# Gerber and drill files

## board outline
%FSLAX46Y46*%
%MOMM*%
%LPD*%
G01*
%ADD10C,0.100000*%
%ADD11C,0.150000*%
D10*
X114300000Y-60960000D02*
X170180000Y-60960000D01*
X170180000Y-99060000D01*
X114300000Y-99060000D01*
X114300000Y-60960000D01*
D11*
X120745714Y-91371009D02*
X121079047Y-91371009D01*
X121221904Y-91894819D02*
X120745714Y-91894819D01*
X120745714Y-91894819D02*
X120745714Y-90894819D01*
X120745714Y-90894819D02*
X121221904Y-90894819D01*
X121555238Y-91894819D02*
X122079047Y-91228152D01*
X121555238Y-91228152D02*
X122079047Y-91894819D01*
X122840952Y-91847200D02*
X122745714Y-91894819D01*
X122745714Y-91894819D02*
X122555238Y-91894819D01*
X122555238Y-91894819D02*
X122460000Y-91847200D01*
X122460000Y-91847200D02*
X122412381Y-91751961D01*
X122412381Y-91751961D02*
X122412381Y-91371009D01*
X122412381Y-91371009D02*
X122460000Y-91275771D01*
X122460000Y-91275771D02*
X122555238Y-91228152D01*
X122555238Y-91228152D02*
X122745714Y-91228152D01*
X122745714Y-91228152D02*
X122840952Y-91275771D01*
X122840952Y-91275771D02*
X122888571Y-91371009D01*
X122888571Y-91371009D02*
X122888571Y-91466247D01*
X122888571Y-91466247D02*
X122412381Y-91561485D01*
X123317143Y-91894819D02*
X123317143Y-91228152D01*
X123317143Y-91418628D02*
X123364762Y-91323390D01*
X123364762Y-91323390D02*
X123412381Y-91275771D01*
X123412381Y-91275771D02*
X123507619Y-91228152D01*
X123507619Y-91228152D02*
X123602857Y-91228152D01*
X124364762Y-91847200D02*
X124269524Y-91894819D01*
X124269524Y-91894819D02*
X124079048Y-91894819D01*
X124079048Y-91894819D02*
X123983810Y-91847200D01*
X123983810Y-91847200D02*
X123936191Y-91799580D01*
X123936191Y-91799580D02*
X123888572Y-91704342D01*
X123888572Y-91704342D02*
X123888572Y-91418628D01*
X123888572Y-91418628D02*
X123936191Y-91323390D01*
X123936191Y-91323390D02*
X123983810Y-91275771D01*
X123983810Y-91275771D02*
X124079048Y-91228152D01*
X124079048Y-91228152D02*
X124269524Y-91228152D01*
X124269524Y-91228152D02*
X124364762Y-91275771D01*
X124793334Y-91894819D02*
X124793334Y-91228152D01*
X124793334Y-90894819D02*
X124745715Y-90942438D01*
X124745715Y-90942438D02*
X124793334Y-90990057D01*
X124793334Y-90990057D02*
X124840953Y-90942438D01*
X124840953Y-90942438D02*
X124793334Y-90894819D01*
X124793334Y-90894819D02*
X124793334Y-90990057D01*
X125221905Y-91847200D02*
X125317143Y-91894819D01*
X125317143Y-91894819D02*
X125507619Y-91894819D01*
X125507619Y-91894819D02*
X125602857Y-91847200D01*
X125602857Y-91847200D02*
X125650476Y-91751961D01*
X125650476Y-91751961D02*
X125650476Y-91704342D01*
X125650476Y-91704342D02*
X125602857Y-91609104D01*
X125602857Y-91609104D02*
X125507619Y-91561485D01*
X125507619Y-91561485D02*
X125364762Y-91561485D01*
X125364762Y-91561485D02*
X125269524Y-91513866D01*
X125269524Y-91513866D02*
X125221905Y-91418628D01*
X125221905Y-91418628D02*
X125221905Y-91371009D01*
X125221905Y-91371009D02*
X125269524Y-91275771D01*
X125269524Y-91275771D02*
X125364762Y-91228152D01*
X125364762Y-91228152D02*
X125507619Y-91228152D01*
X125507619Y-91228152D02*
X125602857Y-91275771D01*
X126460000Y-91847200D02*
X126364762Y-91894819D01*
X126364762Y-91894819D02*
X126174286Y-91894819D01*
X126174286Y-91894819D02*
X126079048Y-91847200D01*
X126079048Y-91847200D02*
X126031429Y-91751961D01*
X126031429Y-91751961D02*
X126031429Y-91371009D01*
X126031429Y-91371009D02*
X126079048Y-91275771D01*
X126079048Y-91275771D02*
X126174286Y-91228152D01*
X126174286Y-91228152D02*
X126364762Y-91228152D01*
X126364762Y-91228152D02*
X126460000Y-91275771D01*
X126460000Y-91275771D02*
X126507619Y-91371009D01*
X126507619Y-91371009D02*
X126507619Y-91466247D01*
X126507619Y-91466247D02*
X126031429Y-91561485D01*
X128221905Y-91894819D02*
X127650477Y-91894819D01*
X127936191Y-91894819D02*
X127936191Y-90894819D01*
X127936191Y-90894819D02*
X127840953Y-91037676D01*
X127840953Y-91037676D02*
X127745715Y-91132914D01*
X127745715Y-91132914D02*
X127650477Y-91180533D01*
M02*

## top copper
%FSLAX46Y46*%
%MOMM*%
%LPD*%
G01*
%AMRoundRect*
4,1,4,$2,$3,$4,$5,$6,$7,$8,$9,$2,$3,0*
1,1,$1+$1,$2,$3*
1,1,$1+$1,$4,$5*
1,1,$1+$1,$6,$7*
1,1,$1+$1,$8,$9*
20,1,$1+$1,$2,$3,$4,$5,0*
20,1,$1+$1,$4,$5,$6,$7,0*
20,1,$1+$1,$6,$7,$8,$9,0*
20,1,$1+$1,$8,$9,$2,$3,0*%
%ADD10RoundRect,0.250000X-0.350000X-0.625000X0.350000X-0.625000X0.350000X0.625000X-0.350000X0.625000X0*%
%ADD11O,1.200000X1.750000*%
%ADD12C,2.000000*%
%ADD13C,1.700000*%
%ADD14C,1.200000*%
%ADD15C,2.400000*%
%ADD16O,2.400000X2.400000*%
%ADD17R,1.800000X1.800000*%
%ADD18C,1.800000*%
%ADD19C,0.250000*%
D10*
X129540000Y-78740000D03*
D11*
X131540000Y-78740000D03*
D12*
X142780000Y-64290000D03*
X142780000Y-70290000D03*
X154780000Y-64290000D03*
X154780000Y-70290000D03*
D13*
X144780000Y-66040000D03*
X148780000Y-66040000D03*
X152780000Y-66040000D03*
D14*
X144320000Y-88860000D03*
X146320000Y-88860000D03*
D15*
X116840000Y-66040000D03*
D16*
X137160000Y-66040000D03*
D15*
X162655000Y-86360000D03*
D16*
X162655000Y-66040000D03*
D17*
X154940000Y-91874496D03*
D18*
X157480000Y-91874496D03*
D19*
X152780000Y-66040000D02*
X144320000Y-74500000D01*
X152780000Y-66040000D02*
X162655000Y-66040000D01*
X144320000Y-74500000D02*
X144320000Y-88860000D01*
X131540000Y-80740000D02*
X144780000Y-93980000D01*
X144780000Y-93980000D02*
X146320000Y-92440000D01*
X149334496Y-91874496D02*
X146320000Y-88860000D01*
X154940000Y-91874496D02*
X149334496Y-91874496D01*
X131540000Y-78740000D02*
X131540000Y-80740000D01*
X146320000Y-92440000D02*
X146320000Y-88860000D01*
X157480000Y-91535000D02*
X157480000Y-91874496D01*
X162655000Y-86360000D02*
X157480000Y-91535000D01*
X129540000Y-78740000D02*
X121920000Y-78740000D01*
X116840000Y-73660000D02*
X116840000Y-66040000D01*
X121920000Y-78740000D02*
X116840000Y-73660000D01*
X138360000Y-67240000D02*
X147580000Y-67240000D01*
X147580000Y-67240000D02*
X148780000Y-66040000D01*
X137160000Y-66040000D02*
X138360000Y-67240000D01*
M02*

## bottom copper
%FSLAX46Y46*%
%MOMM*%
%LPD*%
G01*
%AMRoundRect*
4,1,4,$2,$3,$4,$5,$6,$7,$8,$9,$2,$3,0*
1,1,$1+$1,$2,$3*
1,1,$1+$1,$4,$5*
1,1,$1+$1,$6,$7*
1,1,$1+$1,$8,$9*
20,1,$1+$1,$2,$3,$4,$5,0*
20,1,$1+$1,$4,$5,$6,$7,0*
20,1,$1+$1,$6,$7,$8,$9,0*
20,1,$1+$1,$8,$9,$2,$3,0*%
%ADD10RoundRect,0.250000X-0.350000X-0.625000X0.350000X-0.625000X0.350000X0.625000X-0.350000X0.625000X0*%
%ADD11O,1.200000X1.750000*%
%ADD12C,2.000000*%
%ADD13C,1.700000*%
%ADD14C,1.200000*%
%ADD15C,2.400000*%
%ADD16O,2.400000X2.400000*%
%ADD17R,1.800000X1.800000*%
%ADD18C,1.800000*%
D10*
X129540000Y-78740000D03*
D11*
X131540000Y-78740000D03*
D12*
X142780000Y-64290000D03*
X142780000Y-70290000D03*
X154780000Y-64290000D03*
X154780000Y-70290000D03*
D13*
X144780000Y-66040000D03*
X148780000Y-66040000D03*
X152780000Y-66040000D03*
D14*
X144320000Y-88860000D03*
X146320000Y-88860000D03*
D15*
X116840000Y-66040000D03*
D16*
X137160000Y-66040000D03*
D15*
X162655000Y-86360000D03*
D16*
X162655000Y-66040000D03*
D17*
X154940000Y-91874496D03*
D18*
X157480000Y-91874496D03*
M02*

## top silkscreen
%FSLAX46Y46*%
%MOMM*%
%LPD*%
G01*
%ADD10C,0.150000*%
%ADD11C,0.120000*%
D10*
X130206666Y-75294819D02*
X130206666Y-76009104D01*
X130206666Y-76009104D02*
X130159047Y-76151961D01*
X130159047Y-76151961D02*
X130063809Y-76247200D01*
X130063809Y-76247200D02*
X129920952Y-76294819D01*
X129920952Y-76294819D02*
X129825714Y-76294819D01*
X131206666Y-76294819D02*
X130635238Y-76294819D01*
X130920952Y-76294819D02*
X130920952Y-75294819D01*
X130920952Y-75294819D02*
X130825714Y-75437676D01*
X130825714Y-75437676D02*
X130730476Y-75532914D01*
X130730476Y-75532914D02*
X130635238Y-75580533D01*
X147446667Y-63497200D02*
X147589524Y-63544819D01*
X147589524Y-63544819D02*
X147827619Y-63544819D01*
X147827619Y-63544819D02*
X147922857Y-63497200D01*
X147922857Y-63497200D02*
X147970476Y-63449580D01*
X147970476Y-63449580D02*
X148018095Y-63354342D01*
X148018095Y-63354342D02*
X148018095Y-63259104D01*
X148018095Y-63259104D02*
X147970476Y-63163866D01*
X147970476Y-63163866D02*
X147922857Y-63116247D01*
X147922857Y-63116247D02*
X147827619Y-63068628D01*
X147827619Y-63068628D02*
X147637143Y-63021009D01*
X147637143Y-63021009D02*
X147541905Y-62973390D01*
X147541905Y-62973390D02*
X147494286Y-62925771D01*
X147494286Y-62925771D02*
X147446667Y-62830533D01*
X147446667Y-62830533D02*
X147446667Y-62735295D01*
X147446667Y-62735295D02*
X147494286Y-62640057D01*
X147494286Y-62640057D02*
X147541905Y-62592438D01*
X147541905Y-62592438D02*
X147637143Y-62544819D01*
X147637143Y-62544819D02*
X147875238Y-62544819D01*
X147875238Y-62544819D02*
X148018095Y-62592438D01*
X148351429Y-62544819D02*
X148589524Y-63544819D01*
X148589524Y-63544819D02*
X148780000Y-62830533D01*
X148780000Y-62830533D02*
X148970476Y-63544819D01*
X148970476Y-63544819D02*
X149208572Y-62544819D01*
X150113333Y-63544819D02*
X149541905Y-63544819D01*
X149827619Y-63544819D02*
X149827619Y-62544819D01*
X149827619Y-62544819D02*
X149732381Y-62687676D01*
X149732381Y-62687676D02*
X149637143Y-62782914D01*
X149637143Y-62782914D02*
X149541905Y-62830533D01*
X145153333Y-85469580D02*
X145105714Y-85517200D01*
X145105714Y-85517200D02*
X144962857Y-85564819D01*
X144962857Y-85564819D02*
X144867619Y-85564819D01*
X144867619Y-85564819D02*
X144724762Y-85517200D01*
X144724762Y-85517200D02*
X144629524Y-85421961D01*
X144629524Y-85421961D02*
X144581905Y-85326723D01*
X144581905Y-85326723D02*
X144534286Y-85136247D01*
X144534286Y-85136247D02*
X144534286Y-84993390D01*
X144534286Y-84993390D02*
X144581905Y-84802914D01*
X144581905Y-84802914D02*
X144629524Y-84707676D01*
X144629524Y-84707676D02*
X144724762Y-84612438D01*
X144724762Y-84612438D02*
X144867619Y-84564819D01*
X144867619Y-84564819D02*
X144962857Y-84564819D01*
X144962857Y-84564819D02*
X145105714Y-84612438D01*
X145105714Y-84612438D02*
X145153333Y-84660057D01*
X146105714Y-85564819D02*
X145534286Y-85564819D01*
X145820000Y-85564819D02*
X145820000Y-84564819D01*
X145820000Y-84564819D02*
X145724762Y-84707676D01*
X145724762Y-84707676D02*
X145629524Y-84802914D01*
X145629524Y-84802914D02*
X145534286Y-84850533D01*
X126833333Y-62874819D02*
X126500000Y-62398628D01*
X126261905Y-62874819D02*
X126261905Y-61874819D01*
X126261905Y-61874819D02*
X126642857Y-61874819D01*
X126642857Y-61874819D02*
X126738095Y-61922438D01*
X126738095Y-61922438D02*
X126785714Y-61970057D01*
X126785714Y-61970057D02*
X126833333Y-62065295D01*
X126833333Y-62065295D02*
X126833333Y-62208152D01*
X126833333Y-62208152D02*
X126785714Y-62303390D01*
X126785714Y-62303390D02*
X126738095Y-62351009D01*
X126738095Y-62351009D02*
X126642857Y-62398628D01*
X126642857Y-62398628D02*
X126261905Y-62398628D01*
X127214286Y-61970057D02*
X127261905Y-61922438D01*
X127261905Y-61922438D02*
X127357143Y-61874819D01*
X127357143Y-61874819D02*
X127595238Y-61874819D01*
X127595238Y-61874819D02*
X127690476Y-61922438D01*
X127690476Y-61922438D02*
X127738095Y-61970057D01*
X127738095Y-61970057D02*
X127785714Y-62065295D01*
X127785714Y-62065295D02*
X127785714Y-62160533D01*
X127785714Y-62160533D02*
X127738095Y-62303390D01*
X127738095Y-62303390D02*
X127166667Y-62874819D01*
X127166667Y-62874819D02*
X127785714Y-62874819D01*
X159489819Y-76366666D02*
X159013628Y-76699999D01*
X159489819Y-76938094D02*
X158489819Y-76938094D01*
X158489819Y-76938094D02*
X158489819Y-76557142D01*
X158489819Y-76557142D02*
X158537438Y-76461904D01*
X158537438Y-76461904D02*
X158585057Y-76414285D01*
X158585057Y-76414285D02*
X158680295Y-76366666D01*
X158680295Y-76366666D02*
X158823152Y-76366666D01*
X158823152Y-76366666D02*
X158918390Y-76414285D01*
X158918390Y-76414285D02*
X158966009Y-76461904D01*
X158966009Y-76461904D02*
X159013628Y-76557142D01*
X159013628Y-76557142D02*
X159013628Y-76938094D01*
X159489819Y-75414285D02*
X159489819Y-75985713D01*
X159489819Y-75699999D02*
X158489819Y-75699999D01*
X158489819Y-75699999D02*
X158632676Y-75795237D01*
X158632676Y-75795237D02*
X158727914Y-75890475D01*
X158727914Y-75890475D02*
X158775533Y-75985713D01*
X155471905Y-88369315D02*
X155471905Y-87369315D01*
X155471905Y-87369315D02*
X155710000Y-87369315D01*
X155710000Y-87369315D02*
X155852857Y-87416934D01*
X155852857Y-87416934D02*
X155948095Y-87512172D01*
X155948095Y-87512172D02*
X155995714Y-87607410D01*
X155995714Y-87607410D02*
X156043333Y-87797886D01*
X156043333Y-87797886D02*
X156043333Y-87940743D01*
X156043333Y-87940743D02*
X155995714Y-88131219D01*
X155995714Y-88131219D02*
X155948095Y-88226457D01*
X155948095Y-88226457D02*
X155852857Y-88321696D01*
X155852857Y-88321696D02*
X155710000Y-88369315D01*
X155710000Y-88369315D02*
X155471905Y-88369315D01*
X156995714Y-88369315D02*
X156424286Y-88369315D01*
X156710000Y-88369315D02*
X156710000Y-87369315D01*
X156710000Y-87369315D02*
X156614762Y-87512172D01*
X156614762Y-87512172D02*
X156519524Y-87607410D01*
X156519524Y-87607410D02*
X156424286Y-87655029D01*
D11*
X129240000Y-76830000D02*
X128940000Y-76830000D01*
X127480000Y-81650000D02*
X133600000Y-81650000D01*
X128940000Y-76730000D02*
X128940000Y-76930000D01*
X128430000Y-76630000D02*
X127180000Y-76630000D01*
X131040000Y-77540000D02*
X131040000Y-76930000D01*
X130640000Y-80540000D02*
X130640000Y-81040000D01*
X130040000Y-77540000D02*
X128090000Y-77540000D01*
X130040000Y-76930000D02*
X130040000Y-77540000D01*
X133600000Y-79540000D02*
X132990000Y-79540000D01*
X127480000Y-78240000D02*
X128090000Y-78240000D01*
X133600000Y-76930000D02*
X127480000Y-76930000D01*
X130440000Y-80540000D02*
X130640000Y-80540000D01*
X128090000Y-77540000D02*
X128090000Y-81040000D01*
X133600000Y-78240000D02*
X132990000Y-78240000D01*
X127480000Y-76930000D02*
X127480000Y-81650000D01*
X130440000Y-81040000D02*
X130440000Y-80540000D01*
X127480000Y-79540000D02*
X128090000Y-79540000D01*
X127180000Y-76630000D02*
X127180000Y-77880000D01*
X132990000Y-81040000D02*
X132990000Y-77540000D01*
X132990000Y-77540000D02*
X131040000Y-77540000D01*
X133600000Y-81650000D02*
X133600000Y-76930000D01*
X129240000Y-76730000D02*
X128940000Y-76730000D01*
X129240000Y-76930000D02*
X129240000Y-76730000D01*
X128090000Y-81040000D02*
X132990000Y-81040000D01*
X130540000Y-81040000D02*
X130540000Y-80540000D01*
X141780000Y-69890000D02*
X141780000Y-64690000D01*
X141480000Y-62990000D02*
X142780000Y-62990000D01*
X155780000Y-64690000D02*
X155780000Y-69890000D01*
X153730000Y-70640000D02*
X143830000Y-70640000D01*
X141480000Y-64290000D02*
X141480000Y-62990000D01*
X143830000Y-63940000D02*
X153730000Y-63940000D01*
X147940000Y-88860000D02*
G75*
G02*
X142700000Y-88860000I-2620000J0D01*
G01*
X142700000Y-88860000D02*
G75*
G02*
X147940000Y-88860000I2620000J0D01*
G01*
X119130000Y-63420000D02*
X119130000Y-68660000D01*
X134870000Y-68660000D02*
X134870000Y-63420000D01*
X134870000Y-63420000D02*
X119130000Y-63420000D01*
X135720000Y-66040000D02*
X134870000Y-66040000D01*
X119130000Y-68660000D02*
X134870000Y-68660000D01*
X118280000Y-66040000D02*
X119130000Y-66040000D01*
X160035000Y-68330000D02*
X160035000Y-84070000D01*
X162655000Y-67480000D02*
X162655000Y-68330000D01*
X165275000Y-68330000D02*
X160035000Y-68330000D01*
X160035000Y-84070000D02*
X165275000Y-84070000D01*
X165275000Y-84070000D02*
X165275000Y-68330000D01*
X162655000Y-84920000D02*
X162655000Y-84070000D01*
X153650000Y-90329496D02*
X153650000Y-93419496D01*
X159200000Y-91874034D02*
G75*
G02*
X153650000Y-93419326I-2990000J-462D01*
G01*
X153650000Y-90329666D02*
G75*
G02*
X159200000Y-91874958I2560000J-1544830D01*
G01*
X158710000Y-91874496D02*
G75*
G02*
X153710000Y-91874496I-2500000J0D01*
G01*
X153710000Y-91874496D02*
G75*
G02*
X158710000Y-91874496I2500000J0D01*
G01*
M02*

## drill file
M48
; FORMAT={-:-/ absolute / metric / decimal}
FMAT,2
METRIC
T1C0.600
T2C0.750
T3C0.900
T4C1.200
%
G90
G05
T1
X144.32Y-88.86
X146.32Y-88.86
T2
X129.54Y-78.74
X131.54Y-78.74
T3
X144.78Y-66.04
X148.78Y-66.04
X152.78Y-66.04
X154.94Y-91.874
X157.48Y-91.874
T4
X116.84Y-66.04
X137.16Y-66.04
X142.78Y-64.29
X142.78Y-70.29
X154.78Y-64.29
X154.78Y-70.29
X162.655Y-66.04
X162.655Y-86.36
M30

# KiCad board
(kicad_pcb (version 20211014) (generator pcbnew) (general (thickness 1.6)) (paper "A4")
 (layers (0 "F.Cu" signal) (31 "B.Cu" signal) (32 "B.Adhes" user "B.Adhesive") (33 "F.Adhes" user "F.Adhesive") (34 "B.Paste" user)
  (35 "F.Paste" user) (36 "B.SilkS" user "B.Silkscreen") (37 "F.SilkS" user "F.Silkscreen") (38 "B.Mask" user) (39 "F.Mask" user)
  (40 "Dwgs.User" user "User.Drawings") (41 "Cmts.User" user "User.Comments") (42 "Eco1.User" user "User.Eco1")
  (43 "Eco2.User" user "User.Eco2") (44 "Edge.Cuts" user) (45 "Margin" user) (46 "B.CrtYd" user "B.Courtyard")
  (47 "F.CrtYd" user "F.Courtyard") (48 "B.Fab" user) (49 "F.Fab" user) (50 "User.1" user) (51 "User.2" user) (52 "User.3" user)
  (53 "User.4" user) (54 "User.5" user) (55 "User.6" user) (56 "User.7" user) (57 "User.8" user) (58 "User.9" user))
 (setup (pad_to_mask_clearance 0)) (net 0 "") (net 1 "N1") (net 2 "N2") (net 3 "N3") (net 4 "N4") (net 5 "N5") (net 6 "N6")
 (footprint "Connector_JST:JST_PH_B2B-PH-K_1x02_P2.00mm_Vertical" (layer "F.Cu") (at 129.54 78.74)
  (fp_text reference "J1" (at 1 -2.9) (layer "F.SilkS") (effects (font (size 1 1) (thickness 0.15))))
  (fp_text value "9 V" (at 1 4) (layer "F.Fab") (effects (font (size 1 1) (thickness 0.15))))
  (fp_line (start -0.3 -1.91) (end -0.6 -1.91) (layer "F.SilkS") (width 0.12))
  (fp_line (start -2.06 2.91) (end 4.06 2.91) (layer "F.SilkS") (width 0.12))
  (fp_line (start -0.6 -2.01) (end -0.6 -1.81) (layer "F.SilkS") (width 0.12))
  (fp_line (start -1.11 -2.11) (end -2.36 -2.11) (layer "F.SilkS") (width 0.12))
  (fp_line (start 1.5 -1.2) (end 1.5 -1.81) (layer "F.SilkS") (width 0.12))
  (fp_line (start 1.1 1.8) (end 1.1 2.3) (layer "F.SilkS") (width 0.12))
  (fp_line (start 0.5 -1.2) (end -1.45 -1.2) (layer "F.SilkS") (width 0.12))
  (fp_line (start 0.5 -1.81) (end 0.5 -1.2) (layer "F.SilkS") (width 0.12))
  (fp_line (start 4.06 0.8) (end 3.45 0.8) (layer "F.SilkS") (width 0.12))
  (fp_line (start -2.06 -0.5) (end -1.45 -0.5) (layer "F.SilkS") (width 0.12))
  (fp_line (start 4.06 -1.81) (end -2.06 -1.81) (layer "F.SilkS") (width 0.12))
  (fp_line (start 0.9 1.8) (end 1.1 1.8) (layer "F.SilkS") (width 0.12))
  (fp_line (start -1.45 -1.2) (end -1.45 2.3) (layer "F.SilkS") (width 0.12))
  (fp_line (start 4.06 -0.5) (end 3.45 -0.5) (layer "F.SilkS") (width 0.12))
  (fp_line (start -2.06 -1.81) (end -2.06 2.91) (layer "F.SilkS") (width 0.12))
  (fp_line (start 0.9 2.3) (end 0.9 1.8) (layer "F.SilkS") (width 0.12))
  (fp_line (start -2.06 0.8) (end -1.45 0.8) (layer "F.SilkS") (width 0.12))
  (fp_line (start -2.36 -2.11) (end -2.36 -0.86) (layer "F.SilkS") (width 0.12))
  (fp_line (start 3.45 2.3) (end 3.45 -1.2) (layer "F.SilkS") (width 0.12))
  (fp_line (start 3.45 -1.2) (end 1.5 -1.2) (layer "F.SilkS") (width 0.12))
  (fp_line (start 4.06 2.91) (end 4.06 -1.81) (layer "F.SilkS") (width 0.12))
  (fp_line (start -0.3 -2.01) (end -0.6 -2.01) (layer "F.SilkS") (width 0.12))
  (fp_line (start -0.3 -1.81) (end -0.3 -2.01) (layer "F.SilkS") (width 0.12))
  (fp_line (start -1.45 2.3) (end 3.45 2.3) (layer "F.SilkS") (width 0.12))
  (fp_line (start 1 2.3) (end 1 1.8) (layer "F.SilkS") (width 0.12))
  (pad "1" thru_hole roundrect (at 0 0) (size 1.2 1.75) (drill 0.75) (layers *.Cu *.Mask) (roundrect_rratio 0.208333) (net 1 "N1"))
  (pad "2" thru_hole oval (at 2 0) (size 1.2 1.75) (drill 0.75) (layers *.Cu *.Mask) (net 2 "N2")))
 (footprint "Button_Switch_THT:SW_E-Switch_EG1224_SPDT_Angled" (layer "F.Cu") (at 144.78 66.04)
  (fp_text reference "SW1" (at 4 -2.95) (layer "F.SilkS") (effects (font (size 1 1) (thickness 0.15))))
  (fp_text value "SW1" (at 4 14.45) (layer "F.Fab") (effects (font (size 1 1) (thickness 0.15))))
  (fp_line (start -3 3.85) (end -3 -1.35) (layer "F.SilkS") (width 0.12))
  (fp_line (start -3.3 -3.05) (end -2 -3.05) (layer "F.SilkS") (width 0.12))
  (fp_line (start 11 -1.35) (end 11 3.85) (layer "F.SilkS") (width 0.12))
  (fp_line (start 8.95 4.6) (end -0.95 4.6) (layer "F.SilkS") (width 0.12))
  (fp_line (start -3.3 -1.75) (end -3.3 -3.05) (layer "F.SilkS") (width 0.12))
  (fp_line (start -0.95 -2.1) (end 8.95 -2.1) (layer "F.SilkS") (width 0.12))
  (pad "" thru_hole circle (at -2 -1.75) (size 2 2) (drill 1.2) (layers *.Cu *.Mask))
  (pad "" thru_hole circle (at -2 4.25) (size 2 2) (drill 1.2) (layers *.Cu *.Mask))
  (pad "" thru_hole circle (at 10 -1.75) (size 2 2) (drill 1.2) (layers *.Cu *.Mask))
  (pad "" thru_hole circle (at 10 4.25) (size 2 2) (drill 1.2) (layers *.Cu *.Mask))
  (pad "1" thru_hole circle (at 0 0) (size 1.7 1.7) (drill 0.9) (layers *.Cu *.Mask) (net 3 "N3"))
  (pad "2" thru_hole circle (at 4 0) (size 1.7 1.7) (drill 0.9) (layers *.Cu *.Mask) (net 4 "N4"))
  (pad "3" thru_hole circle (at 8 0) (size 1.7 1.7) (drill 0.9) (layers *.Cu *.Mask) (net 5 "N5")))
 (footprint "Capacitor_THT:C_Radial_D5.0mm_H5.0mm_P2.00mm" (layer "F.Cu") (at 144.32 88.86)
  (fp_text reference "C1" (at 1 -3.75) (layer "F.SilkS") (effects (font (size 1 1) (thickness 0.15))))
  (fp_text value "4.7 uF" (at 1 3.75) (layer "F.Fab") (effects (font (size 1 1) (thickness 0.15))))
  (fp_circle (center 1 0) (end 3.62 0) (layer "F.SilkS") (width 0.12) (fill none))
  (pad "1" thru_hole circle (at 0 0) (size 1.2 1.2) (drill 0.6) (layers *.Cu *.Mask) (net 5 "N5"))
  (pad "2" thru_hole circle (at 2 0) (size 1.2 1.2) (drill 0.6) (layers *.Cu *.Mask) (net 2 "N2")))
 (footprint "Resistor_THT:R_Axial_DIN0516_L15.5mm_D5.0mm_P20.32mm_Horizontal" (layer "F.Cu") (at 116.84 66.04)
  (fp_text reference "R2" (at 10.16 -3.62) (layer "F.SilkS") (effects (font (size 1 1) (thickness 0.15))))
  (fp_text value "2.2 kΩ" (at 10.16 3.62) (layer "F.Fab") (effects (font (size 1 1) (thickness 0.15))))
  (fp_line (start 2.29 -2.62) (end 2.29 2.62) (layer "F.SilkS") (width 0.12))
  (fp_line (start 18.03 2.62) (end 18.03 -2.62) (layer "F.SilkS") (width 0.12))
  (fp_line (start 18.03 -2.62) (end 2.29 -2.62) (layer "F.SilkS") (width 0.12))
  (fp_line (start 18.88 0) (end 18.03 0) (layer "F.SilkS") (width 0.12))
  (fp_line (start 2.29 2.62) (end 18.03 2.62) (layer "F.SilkS") (width 0.12))
  (fp_line (start 1.44 0) (end 2.29 0) (layer "F.SilkS") (width 0.12))
  (pad "1" thru_hole circle (at 0 0) (size 2.4 2.4) (drill 1.2) (layers *.Cu *.Mask) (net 1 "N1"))
  (pad "2" thru_hole oval (at 20.32 0) (size 2.4 2.4) (drill 1.2) (layers *.Cu *.Mask) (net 4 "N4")))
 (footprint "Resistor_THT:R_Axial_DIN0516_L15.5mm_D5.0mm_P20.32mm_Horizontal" (layer "F.Cu") (at 162.655 86.36 90)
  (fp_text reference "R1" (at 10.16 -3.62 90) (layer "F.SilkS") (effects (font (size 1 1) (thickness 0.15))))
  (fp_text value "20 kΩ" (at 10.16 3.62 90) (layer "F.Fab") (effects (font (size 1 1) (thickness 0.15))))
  (fp_line (start 18.03 -2.62) (end 2.29 -2.62) (layer "F.SilkS") (width 0.12))
  (fp_line (start 18.88 0) (end 18.03 0) (layer "F.SilkS") (width 0.12))
  (fp_line (start 18.03 2.62) (end 18.03 -2.62) (layer "F.SilkS") (width 0.12))
  (fp_line (start 2.29 -2.62) (end 2.29 2.62) (layer "F.SilkS") (width 0.12))
  (fp_line (start 2.29 2.62) (end 18.03 2.62) (layer "F.SilkS") (width 0.12))
  (fp_line (start 1.44 0) (end 2.29 0) (layer "F.SilkS") (width 0.12))
  (pad "1" thru_hole circle (at 0 0 90) (size 2.4 2.4) (drill 1.2) (layers *.Cu *.Mask) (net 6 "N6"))
  (pad "2" thru_hole oval (at 20.32 0 90) (size 2.4 2.4) (drill 1.2) (layers *.Cu *.Mask) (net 5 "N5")))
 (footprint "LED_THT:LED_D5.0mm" (layer "F.Cu") (at 154.94 91.874496)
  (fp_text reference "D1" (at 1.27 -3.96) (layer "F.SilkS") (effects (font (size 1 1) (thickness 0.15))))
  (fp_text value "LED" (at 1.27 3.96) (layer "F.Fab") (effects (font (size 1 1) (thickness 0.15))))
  (fp_line (start -1.29 -1.545) (end -1.29 1.545) (layer "F.SilkS") (width 0.12))
  (fp_arc (start 4.26 -0.000462) (mid 2.072002 2.880433) (end -1.29 1.54483) (layer "F.SilkS") (width 0.12))
  (fp_arc (start -1.29 -1.54483) (mid 2.072002 -2.880433) (end 4.26 0.000462) (layer "F.SilkS") (width 0.12))
  (fp_circle (center 1.27 0) (end 3.77 0) (layer "F.SilkS") (width 0.12) (fill none))
  (pad "1" thru_hole rect (at 0 0) (size 1.8 1.8) (drill 0.9) (layers *.Cu *.Mask) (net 2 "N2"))
  (pad "2" thru_hole circle (at 2.54 0) (size 1.8 1.8) (drill 0.9) (layers *.Cu *.Mask) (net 6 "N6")))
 (gr_rect (start 170.18 99.06) (end 170.18 99.06) (layer "Edge.Cuts") (width 0.1) (fill none))
 (gr_rect (start 114.3 60.96) (end 170.18 99.06) (layer "Edge.Cuts") (width 0.1) (fill none))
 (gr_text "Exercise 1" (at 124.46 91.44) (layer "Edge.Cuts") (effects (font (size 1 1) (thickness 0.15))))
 (segment (start 152.78 66.04) (end 144.32 74.5) (width 0.25) (layer "F.Cu") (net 5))
 (segment (start 152.78 66.04) (end 162.655 66.04) (width 0.25) (layer "F.Cu") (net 5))
 (segment (start 144.32 74.5) (end 144.32 88.86) (width 0.25) (layer "F.Cu") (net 5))
 (segment (start 131.54 80.74) (end 144.78 93.98) (width 0.25) (layer "F.Cu") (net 2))
 (segment (start 144.78 93.98) (end 146.32 92.44) (width 0.25) (layer "F.Cu") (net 2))
 (segment (start 149.334496 91.874496) (end 146.32 88.86) (width 0.25) (layer "F.Cu") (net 2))
 (segment (start 154.94 91.874496) (end 149.334496 91.874496) (width 0.25) (layer "F.Cu") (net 2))
 (segment (start 131.54 78.74) (end 131.54 80.74) (width 0.25) (layer "F.Cu") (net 2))
 (segment (start 146.32 92.44) (end 146.32 88.86) (width 0.25) (layer "F.Cu") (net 2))
 (segment (start 157.48 91.535) (end 157.48 91.874496) (width 0.25) (layer "F.Cu") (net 6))
 (segment (start 162.655 86.36) (end 157.48 91.535) (width 0.25) (layer "F.Cu") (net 6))
 (segment (start 129.54 78.74) (end 121.92 78.74) (width 0.25) (layer "F.Cu") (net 1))
 (segment (start 116.84 73.66) (end 116.84 66.04) (width 0.25) (layer "F.Cu") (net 1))
 (segment (start 121.92 78.74) (end 116.84 73.66) (width 0.25) (layer "F.Cu") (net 1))
 (segment (start 138.36 67.24) (end 147.58 67.24) (width 0.25) (layer "F.Cu") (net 4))
 (segment (start 147.58 67.24) (end 148.78 66.04) (width 0.25) (layer "F.Cu") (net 4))
 (segment (start 137.16 66.04) (end 138.36 67.24) (width 0.25) (layer "F.Cu") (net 4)))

